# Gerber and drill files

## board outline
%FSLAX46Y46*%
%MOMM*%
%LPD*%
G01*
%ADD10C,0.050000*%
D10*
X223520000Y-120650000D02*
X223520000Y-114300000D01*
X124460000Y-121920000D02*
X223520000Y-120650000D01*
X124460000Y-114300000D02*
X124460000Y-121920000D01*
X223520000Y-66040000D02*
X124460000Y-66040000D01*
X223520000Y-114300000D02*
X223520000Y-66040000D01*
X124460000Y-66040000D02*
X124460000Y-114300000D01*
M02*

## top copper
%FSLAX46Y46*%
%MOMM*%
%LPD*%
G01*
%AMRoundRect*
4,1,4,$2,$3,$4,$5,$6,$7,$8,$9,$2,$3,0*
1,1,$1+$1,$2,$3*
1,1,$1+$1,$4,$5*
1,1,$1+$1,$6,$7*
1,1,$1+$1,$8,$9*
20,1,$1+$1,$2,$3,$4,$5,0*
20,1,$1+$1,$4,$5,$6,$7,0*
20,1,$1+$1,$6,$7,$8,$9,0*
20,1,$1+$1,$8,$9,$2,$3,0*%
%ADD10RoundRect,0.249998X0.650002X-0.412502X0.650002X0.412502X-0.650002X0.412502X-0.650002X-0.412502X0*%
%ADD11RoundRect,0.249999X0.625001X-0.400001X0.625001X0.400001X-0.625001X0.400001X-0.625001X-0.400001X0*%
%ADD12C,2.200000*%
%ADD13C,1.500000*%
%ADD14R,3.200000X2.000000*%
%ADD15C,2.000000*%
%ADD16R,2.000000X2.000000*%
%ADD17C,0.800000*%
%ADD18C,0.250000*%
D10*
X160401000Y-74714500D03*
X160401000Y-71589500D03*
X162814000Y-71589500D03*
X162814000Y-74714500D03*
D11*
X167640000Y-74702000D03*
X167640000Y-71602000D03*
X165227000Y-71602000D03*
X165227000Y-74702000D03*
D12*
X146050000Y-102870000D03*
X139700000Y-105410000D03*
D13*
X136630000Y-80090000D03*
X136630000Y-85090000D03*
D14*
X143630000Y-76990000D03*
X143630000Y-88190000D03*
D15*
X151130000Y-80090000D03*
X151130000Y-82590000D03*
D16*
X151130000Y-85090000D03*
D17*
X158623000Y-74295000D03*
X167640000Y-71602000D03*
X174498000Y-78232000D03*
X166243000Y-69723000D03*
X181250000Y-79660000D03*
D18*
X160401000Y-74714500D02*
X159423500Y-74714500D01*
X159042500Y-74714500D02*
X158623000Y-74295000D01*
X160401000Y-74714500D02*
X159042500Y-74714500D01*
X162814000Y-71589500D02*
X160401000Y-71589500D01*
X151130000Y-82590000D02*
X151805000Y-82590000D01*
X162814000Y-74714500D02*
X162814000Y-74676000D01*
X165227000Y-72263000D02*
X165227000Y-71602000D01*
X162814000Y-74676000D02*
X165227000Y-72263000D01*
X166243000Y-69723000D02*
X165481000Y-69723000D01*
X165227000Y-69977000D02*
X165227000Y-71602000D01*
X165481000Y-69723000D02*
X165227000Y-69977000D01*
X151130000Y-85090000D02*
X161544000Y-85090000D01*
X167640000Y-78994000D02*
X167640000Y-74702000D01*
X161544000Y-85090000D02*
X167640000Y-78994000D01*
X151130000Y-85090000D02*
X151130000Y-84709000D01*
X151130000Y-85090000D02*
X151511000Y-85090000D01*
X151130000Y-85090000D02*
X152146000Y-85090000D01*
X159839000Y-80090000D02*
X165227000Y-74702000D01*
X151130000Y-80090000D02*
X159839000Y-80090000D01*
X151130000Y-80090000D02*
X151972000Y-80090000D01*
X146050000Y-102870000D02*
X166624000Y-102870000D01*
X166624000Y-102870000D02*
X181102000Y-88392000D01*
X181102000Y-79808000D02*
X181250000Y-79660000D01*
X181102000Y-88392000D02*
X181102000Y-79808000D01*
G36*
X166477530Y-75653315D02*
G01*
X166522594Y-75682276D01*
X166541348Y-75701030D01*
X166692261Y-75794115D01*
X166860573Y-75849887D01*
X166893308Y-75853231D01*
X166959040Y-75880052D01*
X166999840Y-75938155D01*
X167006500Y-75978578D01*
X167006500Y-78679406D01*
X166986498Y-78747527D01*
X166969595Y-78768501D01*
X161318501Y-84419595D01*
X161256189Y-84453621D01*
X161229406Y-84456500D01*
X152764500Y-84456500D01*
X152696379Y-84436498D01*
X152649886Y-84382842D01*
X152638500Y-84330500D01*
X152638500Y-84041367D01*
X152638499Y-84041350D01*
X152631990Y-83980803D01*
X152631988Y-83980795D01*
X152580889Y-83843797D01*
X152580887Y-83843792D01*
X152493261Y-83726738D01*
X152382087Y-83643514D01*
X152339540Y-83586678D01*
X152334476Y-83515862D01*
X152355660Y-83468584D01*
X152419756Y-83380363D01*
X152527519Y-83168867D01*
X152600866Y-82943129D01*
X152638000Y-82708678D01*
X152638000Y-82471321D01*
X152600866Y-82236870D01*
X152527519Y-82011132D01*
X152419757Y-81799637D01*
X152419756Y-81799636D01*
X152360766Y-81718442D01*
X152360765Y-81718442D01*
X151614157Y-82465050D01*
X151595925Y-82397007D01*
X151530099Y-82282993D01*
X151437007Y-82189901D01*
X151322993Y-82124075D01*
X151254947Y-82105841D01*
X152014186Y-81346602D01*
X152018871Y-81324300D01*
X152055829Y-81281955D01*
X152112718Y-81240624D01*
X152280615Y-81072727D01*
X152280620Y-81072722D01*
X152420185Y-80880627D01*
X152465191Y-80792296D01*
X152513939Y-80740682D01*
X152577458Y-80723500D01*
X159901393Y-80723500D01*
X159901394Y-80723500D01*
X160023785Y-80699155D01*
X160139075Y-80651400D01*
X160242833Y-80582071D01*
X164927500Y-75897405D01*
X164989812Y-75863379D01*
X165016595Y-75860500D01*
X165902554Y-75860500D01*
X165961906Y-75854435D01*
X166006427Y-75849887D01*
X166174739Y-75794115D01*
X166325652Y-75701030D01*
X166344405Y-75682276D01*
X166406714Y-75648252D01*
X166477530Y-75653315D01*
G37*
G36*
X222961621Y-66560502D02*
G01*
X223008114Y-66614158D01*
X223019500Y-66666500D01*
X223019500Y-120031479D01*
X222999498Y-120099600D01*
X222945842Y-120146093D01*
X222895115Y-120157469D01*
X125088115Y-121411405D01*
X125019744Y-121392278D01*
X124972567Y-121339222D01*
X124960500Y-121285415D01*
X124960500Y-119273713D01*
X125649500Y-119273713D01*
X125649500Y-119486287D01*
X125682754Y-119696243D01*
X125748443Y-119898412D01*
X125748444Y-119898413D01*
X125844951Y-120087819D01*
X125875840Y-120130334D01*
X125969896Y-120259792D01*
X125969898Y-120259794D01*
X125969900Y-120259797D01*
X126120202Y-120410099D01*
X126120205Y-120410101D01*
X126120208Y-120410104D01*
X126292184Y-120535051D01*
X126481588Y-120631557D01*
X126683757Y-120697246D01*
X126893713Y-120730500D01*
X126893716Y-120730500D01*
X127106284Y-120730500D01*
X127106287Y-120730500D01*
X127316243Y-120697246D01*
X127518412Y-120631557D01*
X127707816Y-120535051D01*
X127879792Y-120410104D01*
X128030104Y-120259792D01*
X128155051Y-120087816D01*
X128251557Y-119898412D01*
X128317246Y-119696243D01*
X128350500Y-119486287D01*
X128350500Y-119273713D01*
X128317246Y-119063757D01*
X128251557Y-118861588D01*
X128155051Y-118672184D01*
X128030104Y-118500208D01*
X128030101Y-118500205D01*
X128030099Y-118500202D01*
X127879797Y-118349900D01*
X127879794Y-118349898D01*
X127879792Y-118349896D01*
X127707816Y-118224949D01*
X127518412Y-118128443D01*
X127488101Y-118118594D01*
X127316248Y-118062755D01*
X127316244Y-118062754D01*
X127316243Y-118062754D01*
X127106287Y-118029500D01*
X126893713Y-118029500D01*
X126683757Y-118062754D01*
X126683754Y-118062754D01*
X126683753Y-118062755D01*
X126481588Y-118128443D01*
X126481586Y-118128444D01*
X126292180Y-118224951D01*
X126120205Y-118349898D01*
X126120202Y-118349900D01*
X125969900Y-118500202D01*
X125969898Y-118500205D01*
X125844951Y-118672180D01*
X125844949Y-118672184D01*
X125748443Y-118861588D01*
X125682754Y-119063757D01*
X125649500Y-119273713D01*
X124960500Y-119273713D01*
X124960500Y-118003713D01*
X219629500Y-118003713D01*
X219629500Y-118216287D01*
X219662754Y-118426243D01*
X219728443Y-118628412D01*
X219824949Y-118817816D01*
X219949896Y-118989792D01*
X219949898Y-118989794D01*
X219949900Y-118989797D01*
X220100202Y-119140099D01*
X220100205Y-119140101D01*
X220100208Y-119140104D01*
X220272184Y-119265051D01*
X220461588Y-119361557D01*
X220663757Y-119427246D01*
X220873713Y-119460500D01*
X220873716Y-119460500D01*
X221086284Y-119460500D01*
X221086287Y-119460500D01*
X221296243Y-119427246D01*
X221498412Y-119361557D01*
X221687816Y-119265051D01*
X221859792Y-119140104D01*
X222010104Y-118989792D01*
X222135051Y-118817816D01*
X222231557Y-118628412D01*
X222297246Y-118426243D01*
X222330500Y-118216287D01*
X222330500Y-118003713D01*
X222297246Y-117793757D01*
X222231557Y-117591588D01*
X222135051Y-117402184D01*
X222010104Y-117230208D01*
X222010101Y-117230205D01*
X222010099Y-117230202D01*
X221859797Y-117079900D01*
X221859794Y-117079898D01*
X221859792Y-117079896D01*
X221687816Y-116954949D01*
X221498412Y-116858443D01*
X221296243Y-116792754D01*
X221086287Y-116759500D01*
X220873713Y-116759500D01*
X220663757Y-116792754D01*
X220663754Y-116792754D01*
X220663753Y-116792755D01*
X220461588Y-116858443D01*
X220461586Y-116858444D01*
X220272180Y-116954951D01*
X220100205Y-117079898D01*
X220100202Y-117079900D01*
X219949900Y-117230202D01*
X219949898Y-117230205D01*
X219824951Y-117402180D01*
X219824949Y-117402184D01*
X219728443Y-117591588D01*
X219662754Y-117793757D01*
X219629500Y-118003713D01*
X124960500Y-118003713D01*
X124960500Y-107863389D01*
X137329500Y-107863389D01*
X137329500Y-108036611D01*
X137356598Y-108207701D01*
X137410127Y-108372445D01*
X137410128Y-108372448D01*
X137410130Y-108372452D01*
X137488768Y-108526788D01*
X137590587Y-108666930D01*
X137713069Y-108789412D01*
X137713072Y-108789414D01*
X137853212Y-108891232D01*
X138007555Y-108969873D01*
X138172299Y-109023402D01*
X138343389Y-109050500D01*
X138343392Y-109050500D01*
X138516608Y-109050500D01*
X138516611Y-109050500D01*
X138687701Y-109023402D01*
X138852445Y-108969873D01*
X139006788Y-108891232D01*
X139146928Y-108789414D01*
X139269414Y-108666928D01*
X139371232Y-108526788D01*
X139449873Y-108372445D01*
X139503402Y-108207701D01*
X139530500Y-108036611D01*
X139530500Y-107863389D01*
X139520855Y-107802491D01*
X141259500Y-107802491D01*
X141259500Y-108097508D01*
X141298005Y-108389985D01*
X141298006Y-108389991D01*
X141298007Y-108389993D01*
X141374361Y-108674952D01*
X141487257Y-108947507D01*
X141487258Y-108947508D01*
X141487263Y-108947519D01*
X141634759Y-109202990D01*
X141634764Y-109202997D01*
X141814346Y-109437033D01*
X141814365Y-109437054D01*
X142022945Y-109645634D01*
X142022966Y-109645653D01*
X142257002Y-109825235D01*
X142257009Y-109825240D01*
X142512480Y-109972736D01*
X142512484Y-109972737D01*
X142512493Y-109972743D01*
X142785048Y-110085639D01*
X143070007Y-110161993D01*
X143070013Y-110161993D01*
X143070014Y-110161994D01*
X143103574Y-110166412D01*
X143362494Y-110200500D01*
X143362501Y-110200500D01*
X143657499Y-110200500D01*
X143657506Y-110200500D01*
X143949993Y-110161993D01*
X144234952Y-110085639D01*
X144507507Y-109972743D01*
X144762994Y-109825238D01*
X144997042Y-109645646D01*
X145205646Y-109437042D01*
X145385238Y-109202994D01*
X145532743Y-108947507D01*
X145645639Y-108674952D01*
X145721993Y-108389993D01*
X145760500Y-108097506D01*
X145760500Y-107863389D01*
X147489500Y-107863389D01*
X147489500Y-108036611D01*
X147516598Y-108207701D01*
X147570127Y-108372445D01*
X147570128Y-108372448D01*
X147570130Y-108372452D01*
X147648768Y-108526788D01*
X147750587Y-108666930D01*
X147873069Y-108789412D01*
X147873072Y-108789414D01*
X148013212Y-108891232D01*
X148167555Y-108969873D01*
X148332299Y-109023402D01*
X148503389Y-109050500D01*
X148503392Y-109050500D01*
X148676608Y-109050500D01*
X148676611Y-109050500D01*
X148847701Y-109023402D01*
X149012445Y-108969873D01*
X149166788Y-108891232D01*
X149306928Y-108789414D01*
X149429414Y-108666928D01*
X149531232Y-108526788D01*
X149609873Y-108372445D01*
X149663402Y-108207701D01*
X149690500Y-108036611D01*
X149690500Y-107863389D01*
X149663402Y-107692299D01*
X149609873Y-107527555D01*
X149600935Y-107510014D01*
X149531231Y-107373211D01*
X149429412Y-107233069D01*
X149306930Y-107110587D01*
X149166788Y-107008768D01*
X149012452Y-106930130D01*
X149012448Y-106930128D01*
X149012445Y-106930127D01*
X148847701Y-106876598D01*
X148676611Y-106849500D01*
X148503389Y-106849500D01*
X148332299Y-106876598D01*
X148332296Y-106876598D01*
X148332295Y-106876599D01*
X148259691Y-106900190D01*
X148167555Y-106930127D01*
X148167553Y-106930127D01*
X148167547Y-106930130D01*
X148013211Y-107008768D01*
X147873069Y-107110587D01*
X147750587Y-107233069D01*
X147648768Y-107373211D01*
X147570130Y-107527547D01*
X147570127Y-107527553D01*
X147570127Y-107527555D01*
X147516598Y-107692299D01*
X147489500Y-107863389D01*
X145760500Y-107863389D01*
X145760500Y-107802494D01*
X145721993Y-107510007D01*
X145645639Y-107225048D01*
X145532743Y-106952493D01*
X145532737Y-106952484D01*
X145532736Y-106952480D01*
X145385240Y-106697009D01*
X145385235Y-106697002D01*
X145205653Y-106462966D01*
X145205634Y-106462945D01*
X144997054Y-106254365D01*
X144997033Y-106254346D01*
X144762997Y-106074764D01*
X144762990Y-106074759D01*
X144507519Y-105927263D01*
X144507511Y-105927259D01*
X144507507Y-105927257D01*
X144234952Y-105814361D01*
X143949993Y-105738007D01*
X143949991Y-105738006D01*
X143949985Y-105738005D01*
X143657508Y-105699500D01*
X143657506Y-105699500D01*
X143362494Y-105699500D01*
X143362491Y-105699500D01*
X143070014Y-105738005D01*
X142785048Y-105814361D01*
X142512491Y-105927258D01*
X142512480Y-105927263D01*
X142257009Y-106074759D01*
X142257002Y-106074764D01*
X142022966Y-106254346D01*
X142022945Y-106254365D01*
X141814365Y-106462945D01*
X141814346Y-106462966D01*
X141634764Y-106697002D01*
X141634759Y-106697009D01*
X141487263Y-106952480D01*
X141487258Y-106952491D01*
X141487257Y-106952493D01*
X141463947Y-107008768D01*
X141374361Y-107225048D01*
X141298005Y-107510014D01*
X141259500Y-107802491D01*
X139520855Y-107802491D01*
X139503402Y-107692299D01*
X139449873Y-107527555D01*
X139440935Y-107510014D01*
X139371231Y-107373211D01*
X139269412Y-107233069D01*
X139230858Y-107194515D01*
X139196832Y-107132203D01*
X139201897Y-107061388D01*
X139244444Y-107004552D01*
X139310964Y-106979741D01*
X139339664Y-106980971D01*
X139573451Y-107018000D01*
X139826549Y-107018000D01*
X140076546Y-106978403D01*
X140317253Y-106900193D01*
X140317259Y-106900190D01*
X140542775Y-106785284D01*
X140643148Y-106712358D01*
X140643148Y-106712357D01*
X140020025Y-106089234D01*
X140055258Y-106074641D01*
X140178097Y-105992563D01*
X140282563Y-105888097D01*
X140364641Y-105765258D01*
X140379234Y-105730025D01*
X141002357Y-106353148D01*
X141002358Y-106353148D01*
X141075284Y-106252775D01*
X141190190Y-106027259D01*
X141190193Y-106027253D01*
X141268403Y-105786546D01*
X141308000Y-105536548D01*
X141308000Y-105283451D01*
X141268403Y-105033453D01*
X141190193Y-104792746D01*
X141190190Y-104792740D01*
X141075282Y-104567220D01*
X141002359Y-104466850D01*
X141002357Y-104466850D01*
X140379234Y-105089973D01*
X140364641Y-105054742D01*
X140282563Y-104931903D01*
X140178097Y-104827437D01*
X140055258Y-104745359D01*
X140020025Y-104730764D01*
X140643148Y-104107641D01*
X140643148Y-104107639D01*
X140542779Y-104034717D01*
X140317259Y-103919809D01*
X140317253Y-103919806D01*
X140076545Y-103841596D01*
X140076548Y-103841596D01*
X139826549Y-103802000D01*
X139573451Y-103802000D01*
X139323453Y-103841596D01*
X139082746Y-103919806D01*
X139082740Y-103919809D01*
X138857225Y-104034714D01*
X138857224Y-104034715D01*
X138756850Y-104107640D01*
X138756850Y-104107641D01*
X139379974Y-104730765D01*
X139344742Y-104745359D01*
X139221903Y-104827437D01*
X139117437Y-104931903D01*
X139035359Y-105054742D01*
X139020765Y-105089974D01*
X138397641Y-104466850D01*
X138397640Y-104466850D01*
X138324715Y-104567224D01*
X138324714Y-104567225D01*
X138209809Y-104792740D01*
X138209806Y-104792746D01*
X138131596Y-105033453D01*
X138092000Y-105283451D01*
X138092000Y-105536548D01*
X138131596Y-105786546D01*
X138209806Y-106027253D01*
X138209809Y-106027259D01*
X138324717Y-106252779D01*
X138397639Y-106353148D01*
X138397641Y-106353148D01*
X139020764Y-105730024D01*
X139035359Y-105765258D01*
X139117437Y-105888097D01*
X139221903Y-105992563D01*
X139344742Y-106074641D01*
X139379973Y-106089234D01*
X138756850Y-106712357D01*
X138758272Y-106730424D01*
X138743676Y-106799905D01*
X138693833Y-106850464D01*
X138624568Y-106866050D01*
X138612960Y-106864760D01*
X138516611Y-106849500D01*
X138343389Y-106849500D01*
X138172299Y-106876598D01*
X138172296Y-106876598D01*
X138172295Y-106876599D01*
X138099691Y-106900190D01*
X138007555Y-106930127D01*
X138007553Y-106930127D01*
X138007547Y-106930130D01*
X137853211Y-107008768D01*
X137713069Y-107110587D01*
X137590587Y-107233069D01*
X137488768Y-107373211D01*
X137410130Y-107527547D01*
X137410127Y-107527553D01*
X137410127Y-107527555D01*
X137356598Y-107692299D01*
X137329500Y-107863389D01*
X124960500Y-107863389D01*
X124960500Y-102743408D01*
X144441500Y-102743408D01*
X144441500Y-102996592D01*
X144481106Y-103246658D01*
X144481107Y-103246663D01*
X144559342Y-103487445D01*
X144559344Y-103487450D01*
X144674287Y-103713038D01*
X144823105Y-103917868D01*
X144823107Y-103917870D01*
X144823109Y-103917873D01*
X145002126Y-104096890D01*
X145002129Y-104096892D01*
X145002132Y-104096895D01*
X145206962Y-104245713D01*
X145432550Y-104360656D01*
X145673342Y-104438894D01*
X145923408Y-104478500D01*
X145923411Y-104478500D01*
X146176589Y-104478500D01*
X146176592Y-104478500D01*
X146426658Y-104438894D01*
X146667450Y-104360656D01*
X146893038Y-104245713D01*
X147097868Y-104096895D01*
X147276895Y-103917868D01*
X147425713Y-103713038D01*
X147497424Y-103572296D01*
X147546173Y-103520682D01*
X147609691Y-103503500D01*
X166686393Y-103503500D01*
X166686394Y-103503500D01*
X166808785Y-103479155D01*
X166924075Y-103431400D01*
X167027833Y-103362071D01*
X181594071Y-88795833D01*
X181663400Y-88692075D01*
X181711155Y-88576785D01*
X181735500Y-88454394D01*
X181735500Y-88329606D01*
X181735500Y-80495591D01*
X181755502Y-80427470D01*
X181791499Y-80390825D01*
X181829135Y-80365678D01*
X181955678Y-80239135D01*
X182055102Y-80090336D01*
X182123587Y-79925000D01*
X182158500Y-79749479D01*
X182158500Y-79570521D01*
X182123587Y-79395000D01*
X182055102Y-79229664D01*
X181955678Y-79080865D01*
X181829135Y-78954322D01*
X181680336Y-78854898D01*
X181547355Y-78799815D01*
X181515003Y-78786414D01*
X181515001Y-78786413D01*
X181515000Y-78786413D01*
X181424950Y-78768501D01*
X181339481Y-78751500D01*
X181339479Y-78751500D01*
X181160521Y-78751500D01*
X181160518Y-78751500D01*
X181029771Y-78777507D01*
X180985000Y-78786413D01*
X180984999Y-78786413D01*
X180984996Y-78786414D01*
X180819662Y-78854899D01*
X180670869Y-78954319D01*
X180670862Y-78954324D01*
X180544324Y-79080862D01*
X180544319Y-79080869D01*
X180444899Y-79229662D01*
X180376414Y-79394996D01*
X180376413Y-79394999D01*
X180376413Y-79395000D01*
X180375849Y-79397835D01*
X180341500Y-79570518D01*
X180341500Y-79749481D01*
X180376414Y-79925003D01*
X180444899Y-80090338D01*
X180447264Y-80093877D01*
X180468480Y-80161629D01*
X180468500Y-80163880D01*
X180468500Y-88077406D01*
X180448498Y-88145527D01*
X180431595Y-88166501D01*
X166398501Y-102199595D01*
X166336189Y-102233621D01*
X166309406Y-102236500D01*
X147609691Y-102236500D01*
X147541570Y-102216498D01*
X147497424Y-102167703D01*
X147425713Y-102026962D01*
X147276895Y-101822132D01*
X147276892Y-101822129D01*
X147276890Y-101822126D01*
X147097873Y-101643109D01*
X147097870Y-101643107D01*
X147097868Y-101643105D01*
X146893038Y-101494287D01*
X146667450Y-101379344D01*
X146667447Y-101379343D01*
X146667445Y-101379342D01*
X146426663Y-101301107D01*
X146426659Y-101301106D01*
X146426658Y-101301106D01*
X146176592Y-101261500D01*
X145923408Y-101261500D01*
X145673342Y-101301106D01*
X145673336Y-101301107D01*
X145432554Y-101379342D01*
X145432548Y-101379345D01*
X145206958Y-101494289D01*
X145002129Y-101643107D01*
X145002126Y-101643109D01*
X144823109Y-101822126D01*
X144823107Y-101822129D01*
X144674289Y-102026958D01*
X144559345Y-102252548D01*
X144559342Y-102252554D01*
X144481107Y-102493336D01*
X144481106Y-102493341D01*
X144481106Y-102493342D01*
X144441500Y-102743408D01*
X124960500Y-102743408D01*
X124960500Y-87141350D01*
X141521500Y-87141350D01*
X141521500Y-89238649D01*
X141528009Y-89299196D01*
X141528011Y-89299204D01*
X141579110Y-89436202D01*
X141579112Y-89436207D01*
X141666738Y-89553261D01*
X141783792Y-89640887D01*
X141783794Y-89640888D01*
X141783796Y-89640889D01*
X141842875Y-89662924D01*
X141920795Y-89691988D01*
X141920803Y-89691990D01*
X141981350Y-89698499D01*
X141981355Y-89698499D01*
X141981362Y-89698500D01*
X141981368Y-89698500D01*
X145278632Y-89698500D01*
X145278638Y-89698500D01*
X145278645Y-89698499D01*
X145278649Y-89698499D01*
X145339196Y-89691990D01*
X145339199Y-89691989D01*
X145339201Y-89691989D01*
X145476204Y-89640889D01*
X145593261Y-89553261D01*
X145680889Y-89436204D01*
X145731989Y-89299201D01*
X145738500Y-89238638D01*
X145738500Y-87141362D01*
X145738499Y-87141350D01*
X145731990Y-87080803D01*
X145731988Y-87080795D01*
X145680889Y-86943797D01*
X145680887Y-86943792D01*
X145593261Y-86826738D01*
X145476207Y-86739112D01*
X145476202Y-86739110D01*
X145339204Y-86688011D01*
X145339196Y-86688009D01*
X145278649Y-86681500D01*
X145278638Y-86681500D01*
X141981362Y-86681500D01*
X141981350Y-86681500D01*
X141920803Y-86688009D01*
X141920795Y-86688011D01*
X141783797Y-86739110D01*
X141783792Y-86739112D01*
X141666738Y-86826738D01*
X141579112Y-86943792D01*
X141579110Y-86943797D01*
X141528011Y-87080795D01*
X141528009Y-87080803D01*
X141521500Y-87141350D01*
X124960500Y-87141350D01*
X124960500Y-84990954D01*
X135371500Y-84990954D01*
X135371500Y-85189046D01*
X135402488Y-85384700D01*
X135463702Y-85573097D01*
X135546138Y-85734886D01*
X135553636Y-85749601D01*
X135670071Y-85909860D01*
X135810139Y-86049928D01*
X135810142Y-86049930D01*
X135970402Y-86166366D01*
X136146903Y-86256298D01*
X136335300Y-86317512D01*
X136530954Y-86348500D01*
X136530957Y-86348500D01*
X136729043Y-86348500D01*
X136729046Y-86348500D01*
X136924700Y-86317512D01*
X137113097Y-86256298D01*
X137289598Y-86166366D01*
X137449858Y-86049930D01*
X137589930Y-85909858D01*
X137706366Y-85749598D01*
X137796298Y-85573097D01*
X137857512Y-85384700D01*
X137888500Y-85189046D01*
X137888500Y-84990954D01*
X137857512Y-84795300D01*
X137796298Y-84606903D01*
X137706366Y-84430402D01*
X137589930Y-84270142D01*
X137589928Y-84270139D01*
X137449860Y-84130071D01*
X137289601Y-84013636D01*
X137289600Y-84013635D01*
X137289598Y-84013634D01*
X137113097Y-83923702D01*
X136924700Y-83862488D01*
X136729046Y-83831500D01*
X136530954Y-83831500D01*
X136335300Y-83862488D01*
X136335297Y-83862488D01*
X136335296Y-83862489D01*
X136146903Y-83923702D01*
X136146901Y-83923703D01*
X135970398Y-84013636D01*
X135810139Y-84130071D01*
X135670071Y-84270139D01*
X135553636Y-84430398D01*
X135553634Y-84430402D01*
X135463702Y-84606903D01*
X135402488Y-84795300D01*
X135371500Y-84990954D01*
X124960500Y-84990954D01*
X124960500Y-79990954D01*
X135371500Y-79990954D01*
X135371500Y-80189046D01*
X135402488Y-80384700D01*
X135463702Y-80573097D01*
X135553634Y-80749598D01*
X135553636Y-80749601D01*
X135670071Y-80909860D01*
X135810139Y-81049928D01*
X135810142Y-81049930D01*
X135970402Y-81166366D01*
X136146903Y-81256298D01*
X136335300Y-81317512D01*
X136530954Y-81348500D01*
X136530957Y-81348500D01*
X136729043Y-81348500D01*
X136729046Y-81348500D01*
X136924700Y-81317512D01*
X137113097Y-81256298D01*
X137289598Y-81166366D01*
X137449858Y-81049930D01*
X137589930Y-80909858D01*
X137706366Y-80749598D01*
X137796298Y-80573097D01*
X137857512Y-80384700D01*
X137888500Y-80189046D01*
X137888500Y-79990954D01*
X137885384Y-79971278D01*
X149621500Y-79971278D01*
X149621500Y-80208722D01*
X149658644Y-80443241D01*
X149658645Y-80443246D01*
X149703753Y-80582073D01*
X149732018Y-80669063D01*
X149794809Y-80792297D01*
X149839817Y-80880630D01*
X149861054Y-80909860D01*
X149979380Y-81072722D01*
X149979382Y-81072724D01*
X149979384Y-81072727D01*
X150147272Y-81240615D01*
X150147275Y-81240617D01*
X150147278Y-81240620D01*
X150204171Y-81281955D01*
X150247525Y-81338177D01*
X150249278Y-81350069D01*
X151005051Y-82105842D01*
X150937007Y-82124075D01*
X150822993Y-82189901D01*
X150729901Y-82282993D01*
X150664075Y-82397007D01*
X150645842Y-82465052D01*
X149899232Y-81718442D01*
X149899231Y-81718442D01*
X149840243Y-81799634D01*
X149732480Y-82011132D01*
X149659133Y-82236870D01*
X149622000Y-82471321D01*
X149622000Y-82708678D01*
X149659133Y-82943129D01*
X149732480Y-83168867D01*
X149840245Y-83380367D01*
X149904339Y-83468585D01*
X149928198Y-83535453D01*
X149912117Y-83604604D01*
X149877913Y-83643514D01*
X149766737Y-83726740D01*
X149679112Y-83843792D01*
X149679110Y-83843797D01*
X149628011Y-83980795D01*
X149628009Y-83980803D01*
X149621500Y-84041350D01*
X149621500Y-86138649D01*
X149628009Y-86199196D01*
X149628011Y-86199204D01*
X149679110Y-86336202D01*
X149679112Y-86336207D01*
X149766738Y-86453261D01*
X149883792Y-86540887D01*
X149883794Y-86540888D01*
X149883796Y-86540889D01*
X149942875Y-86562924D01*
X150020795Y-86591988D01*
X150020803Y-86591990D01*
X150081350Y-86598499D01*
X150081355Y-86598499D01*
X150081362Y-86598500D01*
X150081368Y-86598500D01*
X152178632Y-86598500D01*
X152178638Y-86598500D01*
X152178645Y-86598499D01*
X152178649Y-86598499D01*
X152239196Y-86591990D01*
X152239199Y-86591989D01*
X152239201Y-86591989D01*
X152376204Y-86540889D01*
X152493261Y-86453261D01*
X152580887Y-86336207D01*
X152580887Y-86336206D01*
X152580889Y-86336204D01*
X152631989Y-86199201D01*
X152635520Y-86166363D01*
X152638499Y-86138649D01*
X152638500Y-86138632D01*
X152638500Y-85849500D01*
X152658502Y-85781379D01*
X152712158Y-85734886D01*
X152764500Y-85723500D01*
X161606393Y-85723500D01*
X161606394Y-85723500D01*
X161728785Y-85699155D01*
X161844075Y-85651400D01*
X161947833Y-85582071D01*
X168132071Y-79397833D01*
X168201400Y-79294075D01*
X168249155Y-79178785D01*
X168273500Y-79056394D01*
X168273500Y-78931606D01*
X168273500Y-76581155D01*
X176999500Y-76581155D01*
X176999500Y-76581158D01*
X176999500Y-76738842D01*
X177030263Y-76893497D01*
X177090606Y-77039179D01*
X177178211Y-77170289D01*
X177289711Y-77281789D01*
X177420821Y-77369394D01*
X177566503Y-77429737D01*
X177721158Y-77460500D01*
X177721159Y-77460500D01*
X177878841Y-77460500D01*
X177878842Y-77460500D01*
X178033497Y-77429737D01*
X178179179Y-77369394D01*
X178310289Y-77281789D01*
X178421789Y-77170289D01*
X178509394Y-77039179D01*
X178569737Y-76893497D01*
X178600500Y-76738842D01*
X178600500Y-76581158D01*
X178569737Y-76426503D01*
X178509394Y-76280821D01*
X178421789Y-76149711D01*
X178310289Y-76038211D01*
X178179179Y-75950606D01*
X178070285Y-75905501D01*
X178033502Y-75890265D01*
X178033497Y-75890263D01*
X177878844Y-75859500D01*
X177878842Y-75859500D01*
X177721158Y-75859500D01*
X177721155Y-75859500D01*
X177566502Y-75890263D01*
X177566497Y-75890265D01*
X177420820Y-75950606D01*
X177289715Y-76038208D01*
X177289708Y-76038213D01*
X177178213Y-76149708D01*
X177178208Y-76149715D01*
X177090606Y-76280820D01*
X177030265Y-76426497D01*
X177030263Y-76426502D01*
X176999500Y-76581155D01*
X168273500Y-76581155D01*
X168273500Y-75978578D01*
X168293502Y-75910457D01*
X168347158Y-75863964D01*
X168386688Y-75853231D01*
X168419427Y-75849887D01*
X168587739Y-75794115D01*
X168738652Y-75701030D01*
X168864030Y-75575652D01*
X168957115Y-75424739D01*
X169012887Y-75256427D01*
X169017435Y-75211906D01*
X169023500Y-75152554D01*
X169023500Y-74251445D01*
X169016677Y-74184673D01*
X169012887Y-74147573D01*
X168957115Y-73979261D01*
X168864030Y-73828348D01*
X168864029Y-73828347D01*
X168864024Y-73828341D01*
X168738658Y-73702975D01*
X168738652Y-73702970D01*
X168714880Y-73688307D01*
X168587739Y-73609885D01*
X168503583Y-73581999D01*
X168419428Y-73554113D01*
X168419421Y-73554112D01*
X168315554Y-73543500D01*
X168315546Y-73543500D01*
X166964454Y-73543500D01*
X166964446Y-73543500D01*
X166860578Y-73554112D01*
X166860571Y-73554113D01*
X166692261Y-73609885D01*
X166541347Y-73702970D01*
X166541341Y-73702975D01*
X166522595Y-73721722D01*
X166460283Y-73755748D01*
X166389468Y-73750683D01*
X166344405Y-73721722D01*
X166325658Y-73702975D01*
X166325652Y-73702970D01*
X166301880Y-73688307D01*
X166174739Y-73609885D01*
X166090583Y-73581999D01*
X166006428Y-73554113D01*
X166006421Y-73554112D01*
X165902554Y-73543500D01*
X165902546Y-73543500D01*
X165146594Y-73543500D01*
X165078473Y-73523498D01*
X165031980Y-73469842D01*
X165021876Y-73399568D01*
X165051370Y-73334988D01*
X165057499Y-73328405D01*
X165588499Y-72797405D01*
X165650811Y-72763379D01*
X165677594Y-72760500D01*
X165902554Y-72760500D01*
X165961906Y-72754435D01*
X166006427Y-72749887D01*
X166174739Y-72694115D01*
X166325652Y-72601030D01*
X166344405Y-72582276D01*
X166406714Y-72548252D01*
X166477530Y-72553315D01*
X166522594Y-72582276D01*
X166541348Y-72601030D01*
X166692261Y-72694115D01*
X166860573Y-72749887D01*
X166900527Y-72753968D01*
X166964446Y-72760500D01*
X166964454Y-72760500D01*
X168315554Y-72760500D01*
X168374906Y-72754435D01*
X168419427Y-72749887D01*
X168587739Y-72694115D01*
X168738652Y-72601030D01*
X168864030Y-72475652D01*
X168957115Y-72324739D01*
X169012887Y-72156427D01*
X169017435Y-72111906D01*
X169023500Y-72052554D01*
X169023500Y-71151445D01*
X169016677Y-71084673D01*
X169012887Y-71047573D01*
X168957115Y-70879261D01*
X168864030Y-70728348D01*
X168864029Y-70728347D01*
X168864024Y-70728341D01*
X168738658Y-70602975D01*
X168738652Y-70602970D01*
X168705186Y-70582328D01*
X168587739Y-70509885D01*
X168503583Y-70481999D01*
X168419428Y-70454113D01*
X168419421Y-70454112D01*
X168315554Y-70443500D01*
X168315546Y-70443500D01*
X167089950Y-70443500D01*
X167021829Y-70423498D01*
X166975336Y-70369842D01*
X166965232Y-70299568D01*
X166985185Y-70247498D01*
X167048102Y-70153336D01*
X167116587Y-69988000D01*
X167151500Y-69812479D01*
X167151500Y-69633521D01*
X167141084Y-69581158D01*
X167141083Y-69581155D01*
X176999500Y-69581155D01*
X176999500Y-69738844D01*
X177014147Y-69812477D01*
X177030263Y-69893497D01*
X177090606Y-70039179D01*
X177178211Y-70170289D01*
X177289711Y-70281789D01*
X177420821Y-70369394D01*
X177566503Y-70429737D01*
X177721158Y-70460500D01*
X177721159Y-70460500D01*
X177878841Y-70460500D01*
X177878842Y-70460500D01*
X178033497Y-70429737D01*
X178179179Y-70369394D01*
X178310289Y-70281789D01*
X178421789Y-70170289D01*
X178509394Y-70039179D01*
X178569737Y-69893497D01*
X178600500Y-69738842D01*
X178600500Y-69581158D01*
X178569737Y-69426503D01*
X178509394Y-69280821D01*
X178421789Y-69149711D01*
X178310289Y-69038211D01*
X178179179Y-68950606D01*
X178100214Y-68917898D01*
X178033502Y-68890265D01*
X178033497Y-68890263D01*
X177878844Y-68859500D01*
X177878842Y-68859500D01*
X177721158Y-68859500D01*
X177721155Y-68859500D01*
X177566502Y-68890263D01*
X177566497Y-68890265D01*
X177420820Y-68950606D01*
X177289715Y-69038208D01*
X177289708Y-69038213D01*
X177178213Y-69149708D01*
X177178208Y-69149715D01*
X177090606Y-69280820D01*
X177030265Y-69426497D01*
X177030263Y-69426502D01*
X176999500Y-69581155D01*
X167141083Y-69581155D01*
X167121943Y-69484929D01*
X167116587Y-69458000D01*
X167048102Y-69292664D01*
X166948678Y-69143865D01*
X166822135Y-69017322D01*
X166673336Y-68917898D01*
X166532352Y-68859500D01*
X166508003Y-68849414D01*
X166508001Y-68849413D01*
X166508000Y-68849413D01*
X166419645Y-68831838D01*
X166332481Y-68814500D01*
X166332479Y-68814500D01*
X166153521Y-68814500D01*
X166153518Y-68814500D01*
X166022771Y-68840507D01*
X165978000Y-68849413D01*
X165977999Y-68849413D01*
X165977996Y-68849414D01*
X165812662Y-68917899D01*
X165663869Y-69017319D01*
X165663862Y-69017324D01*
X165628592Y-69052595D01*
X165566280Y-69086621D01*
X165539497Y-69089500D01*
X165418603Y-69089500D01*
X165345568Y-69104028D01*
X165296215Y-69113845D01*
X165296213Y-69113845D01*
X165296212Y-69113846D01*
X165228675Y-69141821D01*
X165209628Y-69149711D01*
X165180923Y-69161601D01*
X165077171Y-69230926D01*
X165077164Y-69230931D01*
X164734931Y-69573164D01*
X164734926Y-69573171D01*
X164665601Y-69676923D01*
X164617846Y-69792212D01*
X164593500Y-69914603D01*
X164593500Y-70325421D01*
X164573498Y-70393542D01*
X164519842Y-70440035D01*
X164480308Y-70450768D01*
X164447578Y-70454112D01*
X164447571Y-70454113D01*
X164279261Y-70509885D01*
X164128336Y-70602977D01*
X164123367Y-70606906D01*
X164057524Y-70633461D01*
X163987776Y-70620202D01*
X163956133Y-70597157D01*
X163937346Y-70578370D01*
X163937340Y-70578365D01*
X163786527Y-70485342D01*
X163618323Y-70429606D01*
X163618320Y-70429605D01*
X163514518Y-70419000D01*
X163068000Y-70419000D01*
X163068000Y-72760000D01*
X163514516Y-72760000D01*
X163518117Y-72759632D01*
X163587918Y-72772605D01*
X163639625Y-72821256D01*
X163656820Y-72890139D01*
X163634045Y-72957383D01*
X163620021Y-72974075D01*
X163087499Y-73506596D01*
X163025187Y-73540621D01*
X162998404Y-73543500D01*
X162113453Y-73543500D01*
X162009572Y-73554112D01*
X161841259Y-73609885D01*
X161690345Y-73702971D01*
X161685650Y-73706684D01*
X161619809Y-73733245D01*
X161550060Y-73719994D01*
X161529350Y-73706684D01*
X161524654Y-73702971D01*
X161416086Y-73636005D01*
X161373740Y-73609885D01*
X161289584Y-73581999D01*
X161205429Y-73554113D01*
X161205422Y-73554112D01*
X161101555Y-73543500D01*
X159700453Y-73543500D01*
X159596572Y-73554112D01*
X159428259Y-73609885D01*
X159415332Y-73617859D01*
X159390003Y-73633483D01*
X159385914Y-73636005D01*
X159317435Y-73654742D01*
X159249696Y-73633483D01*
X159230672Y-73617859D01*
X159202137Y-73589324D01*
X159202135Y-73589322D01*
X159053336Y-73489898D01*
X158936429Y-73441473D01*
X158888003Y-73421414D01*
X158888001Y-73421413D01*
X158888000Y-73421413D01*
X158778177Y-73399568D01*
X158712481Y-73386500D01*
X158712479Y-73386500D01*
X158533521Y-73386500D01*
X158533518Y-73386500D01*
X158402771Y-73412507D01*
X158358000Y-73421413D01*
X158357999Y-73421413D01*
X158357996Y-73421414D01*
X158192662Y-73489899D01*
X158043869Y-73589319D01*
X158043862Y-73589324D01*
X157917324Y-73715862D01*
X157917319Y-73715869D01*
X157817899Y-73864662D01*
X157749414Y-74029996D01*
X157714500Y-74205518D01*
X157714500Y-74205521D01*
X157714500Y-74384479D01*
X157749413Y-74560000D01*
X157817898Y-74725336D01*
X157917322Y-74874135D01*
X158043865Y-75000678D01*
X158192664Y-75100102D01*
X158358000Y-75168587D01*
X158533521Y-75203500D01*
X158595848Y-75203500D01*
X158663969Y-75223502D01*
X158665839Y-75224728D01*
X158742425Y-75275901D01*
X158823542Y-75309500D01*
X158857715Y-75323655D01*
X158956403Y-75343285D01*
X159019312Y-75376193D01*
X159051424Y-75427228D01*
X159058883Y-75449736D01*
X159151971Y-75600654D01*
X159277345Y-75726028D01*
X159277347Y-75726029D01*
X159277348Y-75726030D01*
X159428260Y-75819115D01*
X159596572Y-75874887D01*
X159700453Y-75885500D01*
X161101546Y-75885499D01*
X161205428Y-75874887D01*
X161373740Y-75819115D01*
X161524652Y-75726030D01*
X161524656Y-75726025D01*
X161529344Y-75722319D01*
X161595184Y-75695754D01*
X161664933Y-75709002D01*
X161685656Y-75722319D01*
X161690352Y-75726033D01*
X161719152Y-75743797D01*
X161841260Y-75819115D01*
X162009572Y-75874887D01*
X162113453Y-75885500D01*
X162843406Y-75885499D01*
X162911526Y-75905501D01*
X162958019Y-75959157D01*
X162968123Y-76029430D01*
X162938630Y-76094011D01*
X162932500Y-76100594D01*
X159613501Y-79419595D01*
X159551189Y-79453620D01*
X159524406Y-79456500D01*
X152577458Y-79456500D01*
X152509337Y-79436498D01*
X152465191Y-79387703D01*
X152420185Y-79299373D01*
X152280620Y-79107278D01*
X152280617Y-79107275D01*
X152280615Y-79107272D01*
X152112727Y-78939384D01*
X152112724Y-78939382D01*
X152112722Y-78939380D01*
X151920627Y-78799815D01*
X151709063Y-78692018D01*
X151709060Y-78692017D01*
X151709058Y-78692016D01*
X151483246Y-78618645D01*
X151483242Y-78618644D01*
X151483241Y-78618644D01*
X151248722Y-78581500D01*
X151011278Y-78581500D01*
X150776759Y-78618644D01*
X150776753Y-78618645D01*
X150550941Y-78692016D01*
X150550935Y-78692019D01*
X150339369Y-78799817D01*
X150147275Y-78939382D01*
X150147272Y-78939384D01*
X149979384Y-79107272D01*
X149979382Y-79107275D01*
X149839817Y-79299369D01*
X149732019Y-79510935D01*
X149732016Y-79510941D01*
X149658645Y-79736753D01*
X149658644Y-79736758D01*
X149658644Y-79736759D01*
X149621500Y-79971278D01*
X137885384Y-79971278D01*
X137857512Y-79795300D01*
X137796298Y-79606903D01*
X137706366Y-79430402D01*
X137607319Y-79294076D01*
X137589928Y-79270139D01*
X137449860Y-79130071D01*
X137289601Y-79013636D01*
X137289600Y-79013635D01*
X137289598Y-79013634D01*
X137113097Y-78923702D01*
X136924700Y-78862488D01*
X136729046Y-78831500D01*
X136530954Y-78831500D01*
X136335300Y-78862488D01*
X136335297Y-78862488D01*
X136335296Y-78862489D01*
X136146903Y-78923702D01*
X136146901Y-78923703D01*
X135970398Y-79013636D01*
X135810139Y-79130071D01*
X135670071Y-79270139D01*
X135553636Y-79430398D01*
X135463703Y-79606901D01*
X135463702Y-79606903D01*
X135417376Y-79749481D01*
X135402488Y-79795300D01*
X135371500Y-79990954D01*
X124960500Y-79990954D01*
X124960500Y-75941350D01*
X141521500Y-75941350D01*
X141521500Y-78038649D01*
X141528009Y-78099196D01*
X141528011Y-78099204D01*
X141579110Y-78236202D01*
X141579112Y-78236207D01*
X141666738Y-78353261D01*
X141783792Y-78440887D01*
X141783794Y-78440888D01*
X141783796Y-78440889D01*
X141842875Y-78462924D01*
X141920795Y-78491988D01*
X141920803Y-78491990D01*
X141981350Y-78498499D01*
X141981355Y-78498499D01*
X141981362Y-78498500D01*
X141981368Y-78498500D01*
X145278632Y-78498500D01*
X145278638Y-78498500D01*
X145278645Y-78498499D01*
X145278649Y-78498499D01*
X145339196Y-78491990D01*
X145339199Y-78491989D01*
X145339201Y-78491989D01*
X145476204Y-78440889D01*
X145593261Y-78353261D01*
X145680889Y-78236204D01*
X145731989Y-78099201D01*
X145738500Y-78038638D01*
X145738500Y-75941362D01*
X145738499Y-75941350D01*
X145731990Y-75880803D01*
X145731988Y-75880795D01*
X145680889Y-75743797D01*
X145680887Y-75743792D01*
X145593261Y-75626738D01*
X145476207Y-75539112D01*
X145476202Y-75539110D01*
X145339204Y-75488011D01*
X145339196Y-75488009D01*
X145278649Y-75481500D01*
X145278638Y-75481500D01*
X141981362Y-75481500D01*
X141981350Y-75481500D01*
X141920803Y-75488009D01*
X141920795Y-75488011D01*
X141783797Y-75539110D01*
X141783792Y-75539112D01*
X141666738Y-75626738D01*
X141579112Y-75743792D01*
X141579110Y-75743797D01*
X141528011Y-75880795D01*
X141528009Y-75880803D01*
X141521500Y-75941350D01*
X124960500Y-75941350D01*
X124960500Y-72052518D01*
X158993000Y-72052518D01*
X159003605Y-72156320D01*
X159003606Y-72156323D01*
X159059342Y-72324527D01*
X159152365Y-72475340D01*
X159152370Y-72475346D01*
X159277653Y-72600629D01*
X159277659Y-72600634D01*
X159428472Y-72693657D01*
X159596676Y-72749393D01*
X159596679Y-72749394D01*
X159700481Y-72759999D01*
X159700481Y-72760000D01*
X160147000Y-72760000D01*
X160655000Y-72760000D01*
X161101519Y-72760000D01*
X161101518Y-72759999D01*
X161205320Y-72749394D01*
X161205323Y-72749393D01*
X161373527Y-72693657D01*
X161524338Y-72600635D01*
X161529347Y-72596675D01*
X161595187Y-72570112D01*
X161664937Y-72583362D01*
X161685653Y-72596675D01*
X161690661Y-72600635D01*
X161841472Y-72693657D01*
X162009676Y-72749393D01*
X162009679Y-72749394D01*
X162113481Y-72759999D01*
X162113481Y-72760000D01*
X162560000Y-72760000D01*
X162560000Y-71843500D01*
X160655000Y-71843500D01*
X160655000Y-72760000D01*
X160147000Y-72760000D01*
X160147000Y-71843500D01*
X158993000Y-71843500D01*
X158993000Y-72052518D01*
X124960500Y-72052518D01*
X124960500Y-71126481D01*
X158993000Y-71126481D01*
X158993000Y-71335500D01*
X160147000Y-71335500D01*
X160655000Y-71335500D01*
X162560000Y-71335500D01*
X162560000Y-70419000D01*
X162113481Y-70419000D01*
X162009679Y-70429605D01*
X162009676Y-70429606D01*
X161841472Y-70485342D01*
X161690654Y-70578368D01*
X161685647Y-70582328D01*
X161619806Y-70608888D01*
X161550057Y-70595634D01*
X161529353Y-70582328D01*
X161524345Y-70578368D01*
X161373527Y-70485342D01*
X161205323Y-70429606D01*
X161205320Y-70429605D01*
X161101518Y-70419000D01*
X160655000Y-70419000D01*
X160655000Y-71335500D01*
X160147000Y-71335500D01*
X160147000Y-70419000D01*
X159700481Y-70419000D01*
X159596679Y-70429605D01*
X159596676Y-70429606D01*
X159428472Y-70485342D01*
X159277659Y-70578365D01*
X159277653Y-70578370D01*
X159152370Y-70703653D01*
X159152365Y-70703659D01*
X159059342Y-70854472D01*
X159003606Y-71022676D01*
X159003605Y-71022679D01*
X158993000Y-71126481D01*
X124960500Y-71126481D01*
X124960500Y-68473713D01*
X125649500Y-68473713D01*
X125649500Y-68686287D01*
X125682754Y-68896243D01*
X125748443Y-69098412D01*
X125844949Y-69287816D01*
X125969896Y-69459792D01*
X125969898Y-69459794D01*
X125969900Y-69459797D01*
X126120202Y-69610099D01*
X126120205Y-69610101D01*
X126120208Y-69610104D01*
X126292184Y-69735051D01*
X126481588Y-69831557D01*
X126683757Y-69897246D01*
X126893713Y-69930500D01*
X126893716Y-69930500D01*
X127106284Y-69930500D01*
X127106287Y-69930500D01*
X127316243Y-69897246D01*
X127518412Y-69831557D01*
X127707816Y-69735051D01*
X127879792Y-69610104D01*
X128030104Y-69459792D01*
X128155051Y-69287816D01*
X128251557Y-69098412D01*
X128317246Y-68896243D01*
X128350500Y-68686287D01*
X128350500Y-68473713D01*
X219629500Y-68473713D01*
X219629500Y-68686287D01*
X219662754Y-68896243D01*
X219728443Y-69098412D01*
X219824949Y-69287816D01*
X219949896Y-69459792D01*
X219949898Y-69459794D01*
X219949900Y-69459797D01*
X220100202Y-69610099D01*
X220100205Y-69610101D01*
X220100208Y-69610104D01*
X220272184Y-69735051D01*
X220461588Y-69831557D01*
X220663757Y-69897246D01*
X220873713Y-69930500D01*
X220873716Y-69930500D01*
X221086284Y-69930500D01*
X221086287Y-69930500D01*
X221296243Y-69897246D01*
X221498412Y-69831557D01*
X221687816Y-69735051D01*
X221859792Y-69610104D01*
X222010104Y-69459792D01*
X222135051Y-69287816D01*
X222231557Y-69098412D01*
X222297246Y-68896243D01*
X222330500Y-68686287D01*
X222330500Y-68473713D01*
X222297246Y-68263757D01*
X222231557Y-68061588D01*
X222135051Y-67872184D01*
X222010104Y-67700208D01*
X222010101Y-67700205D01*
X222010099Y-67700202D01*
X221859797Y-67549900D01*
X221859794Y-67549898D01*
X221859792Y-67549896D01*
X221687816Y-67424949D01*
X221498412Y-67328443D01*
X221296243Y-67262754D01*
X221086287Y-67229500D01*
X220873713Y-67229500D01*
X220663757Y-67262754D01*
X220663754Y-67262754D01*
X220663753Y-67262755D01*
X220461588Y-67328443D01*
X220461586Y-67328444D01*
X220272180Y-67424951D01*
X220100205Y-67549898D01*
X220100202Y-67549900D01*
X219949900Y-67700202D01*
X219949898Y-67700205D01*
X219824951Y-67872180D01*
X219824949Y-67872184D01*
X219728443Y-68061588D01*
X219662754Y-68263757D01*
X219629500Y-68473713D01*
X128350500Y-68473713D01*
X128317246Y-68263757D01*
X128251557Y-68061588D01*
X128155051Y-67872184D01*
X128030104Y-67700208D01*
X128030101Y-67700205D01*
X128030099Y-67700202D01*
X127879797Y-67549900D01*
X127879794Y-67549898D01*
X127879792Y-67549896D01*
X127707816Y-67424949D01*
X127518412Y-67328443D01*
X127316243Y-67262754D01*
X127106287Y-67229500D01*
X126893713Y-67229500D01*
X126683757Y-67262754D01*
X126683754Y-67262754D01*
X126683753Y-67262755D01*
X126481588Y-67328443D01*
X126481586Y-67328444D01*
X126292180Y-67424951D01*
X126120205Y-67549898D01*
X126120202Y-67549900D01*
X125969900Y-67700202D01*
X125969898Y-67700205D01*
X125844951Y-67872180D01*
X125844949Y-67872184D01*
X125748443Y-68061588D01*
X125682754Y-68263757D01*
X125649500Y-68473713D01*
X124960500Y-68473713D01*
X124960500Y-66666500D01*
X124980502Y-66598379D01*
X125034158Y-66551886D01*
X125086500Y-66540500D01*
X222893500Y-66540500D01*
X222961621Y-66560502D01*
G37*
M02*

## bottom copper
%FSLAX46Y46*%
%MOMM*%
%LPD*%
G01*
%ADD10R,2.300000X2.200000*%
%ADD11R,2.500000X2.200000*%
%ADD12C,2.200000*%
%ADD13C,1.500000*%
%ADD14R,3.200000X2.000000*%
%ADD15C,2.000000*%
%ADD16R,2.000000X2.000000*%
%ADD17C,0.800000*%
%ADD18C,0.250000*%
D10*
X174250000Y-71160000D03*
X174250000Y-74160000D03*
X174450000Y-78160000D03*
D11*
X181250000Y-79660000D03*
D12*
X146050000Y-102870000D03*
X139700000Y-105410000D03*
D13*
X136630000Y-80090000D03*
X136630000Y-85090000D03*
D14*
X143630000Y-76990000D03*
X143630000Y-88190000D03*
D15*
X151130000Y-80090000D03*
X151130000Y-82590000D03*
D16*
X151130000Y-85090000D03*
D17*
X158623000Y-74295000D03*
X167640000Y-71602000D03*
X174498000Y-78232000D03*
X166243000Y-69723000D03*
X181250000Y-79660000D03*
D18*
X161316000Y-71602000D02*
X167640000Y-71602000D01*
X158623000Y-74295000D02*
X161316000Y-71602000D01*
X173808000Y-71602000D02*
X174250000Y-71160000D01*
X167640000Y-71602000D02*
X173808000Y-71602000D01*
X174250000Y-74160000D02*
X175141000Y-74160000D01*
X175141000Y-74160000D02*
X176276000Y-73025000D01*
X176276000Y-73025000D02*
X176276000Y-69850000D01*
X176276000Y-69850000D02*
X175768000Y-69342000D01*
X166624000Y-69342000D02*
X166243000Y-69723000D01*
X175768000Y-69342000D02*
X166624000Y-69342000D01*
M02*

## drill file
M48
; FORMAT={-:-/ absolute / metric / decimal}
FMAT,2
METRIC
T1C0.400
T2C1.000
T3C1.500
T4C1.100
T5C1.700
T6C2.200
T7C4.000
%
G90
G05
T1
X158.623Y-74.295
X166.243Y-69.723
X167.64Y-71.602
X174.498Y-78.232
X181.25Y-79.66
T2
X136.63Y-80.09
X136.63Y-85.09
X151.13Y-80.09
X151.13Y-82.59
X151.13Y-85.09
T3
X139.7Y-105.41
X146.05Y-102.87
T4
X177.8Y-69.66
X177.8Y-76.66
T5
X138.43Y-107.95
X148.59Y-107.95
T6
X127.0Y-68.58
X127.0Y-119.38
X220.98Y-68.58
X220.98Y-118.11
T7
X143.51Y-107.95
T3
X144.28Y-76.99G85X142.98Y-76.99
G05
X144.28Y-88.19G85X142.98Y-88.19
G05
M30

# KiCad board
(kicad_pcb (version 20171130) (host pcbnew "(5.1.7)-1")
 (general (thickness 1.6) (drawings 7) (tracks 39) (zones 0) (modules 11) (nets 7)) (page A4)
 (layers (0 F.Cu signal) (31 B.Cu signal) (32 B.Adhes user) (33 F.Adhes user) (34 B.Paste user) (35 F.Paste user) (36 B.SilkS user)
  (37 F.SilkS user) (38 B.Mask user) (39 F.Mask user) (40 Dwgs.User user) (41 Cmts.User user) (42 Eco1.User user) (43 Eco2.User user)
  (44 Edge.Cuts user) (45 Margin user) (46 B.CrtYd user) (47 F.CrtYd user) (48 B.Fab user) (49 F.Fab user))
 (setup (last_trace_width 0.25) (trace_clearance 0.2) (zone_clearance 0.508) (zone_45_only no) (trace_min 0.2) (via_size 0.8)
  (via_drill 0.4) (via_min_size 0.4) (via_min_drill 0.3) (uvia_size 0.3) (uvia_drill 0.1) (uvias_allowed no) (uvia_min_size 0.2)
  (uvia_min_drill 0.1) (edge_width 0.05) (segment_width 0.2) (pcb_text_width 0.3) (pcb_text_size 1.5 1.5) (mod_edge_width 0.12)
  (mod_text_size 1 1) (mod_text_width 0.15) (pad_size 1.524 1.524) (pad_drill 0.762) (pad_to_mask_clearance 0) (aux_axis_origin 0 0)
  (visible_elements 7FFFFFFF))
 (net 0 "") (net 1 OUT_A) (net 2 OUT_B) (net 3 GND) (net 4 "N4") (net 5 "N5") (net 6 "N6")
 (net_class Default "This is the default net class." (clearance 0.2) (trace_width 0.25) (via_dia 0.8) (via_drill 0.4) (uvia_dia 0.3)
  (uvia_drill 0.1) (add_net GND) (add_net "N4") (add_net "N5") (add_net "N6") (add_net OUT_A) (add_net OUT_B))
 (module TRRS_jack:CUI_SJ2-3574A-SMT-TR (layer B.Cu) (at 177.8 73.66 270)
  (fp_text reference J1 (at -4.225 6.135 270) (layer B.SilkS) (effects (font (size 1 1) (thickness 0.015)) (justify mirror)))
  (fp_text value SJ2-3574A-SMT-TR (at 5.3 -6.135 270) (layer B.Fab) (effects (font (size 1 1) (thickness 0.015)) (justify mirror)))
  (pad 4 smd rect (at -2.5 3.55 270) (size 2.2 2.3) (layers B.Cu B.Paste B.Mask) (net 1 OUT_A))
  (pad 3 smd rect (at 0.5 3.55 270) (size 2.2 2.3) (layers B.Cu B.Paste B.Mask) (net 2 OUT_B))
  (pad 2 smd rect (at 4.5 3.35 270) (size 2.2 2.3) (layers B.Cu B.Paste B.Mask) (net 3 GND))
  (pad 1 smd rect (at 6 -3.45 270) (size 2.2 2.5) (layers B.Cu B.Paste B.Mask) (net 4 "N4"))
  (pad None np_thru_hole circle (at -4 0 270) (size 1.1 1.1) (drill 1.1) (layers *.Cu *.Mask))
  (pad None np_thru_hole circle (at 3 0 270) (size 1.1 1.1) (drill 1.1) (layers *.Cu *.Mask)))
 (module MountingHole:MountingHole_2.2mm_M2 (layer F.Cu) (at 127 119.38)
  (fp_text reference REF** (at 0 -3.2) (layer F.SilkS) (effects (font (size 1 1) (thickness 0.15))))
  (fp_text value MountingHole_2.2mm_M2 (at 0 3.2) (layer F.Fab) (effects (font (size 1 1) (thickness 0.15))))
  (pad 1 np_thru_hole circle (at 0 0) (size 2.2 2.2) (drill 2.2) (layers *.Cu *.Mask)))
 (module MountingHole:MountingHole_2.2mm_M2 (layer F.Cu) (at 220.98 118.11)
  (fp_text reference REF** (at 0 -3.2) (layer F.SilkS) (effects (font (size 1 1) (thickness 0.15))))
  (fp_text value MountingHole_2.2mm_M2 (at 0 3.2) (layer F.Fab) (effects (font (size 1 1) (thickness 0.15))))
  (pad 1 np_thru_hole circle (at 0 0) (size 2.2 2.2) (drill 2.2) (layers *.Cu *.Mask)))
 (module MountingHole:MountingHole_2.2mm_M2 (layer F.Cu) (at 220.98 68.58)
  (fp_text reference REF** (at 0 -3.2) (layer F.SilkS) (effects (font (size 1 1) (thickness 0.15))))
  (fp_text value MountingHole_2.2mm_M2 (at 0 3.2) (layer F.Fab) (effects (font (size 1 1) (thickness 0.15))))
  (pad 1 np_thru_hole circle (at 0 0) (size 2.2 2.2) (drill 2.2) (layers *.Cu *.Mask)))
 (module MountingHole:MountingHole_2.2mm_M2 (layer F.Cu) (at 127 68.58)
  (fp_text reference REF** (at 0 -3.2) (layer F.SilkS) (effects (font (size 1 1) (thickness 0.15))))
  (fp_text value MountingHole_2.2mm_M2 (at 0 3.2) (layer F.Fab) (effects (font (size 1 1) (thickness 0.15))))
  (pad 1 np_thru_hole circle (at 0 0) (size 2.2 2.2) (drill 2.2) (layers *.Cu *.Mask)))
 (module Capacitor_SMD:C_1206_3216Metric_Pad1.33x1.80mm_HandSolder (layer F.Cu) (at 160.401 73.152 90)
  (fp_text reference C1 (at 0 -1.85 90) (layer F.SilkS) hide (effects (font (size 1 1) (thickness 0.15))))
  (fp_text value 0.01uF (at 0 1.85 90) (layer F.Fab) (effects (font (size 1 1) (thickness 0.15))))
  (pad 1 smd roundrect (at -1.5625 0 90) (size 1.325 1.8) (layers F.Cu F.Paste F.Mask) (roundrect_rratio 0.1886777358490566) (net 1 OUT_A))
  (pad 2 smd roundrect (at 1.5625 0 90) (size 1.325 1.8) (layers F.Cu F.Paste F.Mask) (roundrect_rratio 0.1886777358490566) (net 3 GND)))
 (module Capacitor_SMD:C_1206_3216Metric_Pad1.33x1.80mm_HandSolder (layer F.Cu) (at 162.814 73.152 90)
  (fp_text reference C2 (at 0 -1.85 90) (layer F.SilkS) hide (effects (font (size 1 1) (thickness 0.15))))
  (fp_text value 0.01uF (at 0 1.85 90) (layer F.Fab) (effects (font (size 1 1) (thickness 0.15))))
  (pad 2 smd roundrect (at 1.5625 0 90) (size 1.325 1.8) (layers F.Cu F.Paste F.Mask) (roundrect_rratio 0.1886777358490566) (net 3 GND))
  (pad 1 smd roundrect (at -1.5625 0 90) (size 1.325 1.8) (layers F.Cu F.Paste F.Mask) (roundrect_rratio 0.1886777358490566) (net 2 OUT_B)))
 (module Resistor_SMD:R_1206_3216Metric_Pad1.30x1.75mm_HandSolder (layer F.Cu) (at 167.64 73.152 90)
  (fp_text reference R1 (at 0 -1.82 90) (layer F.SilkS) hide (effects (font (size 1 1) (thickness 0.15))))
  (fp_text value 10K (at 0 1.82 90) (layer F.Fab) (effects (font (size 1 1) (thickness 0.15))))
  (pad 1 smd roundrect (at -1.55 0 90) (size 1.3 1.75) (layers F.Cu F.Paste F.Mask) (roundrect_rratio 0.1923069230769231) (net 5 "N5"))
  (pad 2 smd roundrect (at 1.55 0 90) (size 1.3 1.75) (layers F.Cu F.Paste F.Mask) (roundrect_rratio 0.1923069230769231) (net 1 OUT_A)))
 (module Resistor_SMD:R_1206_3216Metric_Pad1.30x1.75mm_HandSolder (layer F.Cu) (at 165.227 73.152 90)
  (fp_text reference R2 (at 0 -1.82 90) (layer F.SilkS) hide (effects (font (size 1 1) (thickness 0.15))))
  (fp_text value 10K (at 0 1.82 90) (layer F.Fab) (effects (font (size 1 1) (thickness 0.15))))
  (pad 2 smd roundrect (at 1.55 0 90) (size 1.3 1.75) (layers F.Cu F.Paste F.Mask) (roundrect_rratio 0.1923069230769231) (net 2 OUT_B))
  (pad 1 smd roundrect (at -1.55 0 90) (size 1.3 1.75) (layers F.Cu F.Paste F.Mask) (roundrect_rratio 0.1923069230769231) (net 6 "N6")))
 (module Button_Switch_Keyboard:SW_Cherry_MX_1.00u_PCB (layer F.Cu) (at 146.05 102.87)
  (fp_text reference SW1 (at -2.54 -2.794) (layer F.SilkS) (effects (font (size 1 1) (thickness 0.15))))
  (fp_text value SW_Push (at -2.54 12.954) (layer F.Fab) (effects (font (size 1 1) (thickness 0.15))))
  (pad 1 thru_hole circle (at 0 0) (size 2.2 2.2) (drill 1.5) (layers *.Cu *.Mask) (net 4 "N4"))
  (pad 2 thru_hole circle (at -6.35 2.54) (size 2.2 2.2) (drill 1.5) (layers *.Cu *.Mask) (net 3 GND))
  (pad "" np_thru_hole circle (at -2.54 5.08) (size 4 4) (drill 4) (layers *.Cu *.Mask))
  (pad "" np_thru_hole circle (at -7.62 5.08) (size 1.7 1.7) (drill 1.7) (layers *.Cu *.Mask))
  (pad "" np_thru_hole circle (at 2.54 5.08) (size 1.7 1.7) (drill 1.7) (layers *.Cu *.Mask)))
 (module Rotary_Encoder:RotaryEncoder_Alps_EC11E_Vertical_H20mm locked (layer F.Cu) (at 151.13 85.09 180)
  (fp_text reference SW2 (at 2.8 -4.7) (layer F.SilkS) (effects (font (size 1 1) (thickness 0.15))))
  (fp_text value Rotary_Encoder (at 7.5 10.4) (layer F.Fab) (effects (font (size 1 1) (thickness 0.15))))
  (pad "" thru_hole circle (at 14.5 5 180) (size 1.5 1.5) (drill 1) (layers *.Cu *.Mask))
  (pad "" thru_hole circle (at 14.5 0 180) (size 1.5 1.5) (drill 1) (layers *.Cu *.Mask))
  (pad MP thru_hole rect (at 7.5 8.1 180) (size 3.2 2) (drill oval 2.8 1.5) (layers *.Cu *.Mask))
  (pad MP thru_hole rect (at 7.5 -3.1 180) (size 3.2 2) (drill oval 2.8 1.5) (layers *.Cu *.Mask))
  (pad B thru_hole circle (at 0 5 180) (size 2 2) (drill 1) (layers *.Cu *.Mask) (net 6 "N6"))
  (pad C thru_hole circle (at 0 2.5 180) (size 2 2) (drill 1) (layers *.Cu *.Mask) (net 3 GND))
  (pad A thru_hole rect (at 0 0 180) (size 2 2) (drill 1) (layers *.Cu *.Mask) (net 5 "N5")))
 (gr_line (start 223.52 120.65) (end 223.52 114.3) (layer Edge.Cuts) (width 0.05))
 (gr_line (start 124.46 121.92) (end 223.52 120.65) (layer Edge.Cuts) (width 0.05))
 (gr_line (start 124.46 114.3) (end 124.46 121.92) (layer Edge.Cuts) (width 0.05))
 (gr_line (start 223.52 66.04) (end 124.46 66.04) (layer Edge.Cuts) (width 0.05))
 (gr_line (start 223.52 114.3) (end 223.52 66.04) (layer Edge.Cuts) (width 0.05))
 (gr_line (start 124.46 66.04) (end 124.46 114.3) (layer Edge.Cuts) (width 0.05))
 (segment (start 160.401 74.7145) (end 159.4235 74.7145) (width 0.25) (layer F.Cu) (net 1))
 (via (at 158.623 74.295) (size 0.8) (drill 0.4) (layers F.Cu B.Cu) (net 1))
 (segment (start 159.0425 74.7145) (end 158.623 74.295) (width 0.25) (layer F.Cu) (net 1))
 (segment (start 160.401 74.7145) (end 159.0425 74.7145) (width 0.25) (layer F.Cu) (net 1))
 (via (at 167.64 71.602) (size 0.8) (drill 0.4) (layers F.Cu B.Cu) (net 1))
 (segment (start 161.316 71.602) (end 167.64 71.602) (width 0.25) (layer B.Cu) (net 1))
 (segment (start 158.623 74.295) (end 161.316 71.602) (width 0.25) (layer B.Cu) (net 1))
 (segment (start 173.808 71.602) (end 174.25 71.16) (width 0.25) (layer B.Cu) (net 1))
 (segment (start 167.64 71.602) (end 173.808 71.602) (width 0.25) (layer B.Cu) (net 1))
 (via (at 174.498 78.232) (size 0.8) (drill 0.4) (layers F.Cu B.Cu) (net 3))
 (segment (start 162.814 71.5895) (end 160.401 71.5895) (width 0.25) (layer F.Cu) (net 3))
 (segment (start 151.13 82.59) (end 151.805 82.59) (width 0.25) (layer F.Cu) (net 3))
 (segment (start 162.814 74.7145) (end 162.814 74.676) (width 0.25) (layer F.Cu) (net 2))
 (segment (start 165.227 72.263) (end 165.227 71.602) (width 0.25) (layer F.Cu) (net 2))
 (segment (start 162.814 74.676) (end 165.227 72.263) (width 0.25) (layer F.Cu) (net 2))
 (segment (start 174.25 74.16) (end 175.141 74.16) (width 0.25) (layer B.Cu) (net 2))
 (segment (start 175.141 74.16) (end 176.276 73.025) (width 0.25) (layer B.Cu) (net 2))
 (segment (start 176.276 73.025) (end 176.276 69.85) (width 0.25) (layer B.Cu) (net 2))
 (segment (start 176.276 69.85) (end 175.768 69.342) (width 0.25) (layer B.Cu) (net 2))
 (via (at 166.243 69.723) (size 0.8) (drill 0.4) (layers F.Cu B.Cu) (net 2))
 (segment (start 166.624 69.342) (end 166.243 69.723) (width 0.25) (layer B.Cu) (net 2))
 (segment (start 175.768 69.342) (end 166.624 69.342) (width 0.25) (layer B.Cu) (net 2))
 (segment (start 166.243 69.723) (end 165.481 69.723) (width 0.25) (layer F.Cu) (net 2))
 (segment (start 165.227 69.977) (end 165.227 71.602) (width 0.25) (layer F.Cu) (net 2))
 (segment (start 165.481 69.723) (end 165.227 69.977) (width 0.25) (layer F.Cu) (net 2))
 (segment (start 151.13 85.09) (end 161.544 85.09) (width 0.25) (layer F.Cu) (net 5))
 (segment (start 167.64 78.994) (end 167.64 74.702) (width 0.25) (layer F.Cu) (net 5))
 (segment (start 161.544 85.09) (end 167.64 78.994) (width 0.25) (layer F.Cu) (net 5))
 (segment (start 151.13 85.09) (end 151.13 84.709) (width 0.25) (layer F.Cu) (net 5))
 (segment (start 151.13 85.09) (end 151.511 85.09) (width 0.25) (layer F.Cu) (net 5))
 (segment (start 151.13 85.09) (end 152.146 85.09) (width 0.25) (layer F.Cu) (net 5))
 (segment (start 159.839 80.09) (end 165.227 74.702) (width 0.25) (layer F.Cu) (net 6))
 (segment (start 151.13 80.09) (end 159.839 80.09) (width 0.25) (layer F.Cu) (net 6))
 (segment (start 151.13 80.09) (end 151.972 80.09) (width 0.25) (layer F.Cu) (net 6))
 (segment (start 146.05 102.87) (end 166.624 102.87) (width 0.25) (layer F.Cu) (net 4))
 (segment (start 166.624 102.87) (end 181.102 88.392) (width 0.25) (layer F.Cu) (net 4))
 (via (at 181.25 79.66) (size 0.8) (drill 0.4) (layers F.Cu B.Cu) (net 4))
 (segment (start 181.102 79.808) (end 181.25 79.66) (width 0.25) (layer F.Cu) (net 4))
 (segment (start 181.102 88.392) (end 181.102 79.808) (width 0.25) (layer F.Cu) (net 4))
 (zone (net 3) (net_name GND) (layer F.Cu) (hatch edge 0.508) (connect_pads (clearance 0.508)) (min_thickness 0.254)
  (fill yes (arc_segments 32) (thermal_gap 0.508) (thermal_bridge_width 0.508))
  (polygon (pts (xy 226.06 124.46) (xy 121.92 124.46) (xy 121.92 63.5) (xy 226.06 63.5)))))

